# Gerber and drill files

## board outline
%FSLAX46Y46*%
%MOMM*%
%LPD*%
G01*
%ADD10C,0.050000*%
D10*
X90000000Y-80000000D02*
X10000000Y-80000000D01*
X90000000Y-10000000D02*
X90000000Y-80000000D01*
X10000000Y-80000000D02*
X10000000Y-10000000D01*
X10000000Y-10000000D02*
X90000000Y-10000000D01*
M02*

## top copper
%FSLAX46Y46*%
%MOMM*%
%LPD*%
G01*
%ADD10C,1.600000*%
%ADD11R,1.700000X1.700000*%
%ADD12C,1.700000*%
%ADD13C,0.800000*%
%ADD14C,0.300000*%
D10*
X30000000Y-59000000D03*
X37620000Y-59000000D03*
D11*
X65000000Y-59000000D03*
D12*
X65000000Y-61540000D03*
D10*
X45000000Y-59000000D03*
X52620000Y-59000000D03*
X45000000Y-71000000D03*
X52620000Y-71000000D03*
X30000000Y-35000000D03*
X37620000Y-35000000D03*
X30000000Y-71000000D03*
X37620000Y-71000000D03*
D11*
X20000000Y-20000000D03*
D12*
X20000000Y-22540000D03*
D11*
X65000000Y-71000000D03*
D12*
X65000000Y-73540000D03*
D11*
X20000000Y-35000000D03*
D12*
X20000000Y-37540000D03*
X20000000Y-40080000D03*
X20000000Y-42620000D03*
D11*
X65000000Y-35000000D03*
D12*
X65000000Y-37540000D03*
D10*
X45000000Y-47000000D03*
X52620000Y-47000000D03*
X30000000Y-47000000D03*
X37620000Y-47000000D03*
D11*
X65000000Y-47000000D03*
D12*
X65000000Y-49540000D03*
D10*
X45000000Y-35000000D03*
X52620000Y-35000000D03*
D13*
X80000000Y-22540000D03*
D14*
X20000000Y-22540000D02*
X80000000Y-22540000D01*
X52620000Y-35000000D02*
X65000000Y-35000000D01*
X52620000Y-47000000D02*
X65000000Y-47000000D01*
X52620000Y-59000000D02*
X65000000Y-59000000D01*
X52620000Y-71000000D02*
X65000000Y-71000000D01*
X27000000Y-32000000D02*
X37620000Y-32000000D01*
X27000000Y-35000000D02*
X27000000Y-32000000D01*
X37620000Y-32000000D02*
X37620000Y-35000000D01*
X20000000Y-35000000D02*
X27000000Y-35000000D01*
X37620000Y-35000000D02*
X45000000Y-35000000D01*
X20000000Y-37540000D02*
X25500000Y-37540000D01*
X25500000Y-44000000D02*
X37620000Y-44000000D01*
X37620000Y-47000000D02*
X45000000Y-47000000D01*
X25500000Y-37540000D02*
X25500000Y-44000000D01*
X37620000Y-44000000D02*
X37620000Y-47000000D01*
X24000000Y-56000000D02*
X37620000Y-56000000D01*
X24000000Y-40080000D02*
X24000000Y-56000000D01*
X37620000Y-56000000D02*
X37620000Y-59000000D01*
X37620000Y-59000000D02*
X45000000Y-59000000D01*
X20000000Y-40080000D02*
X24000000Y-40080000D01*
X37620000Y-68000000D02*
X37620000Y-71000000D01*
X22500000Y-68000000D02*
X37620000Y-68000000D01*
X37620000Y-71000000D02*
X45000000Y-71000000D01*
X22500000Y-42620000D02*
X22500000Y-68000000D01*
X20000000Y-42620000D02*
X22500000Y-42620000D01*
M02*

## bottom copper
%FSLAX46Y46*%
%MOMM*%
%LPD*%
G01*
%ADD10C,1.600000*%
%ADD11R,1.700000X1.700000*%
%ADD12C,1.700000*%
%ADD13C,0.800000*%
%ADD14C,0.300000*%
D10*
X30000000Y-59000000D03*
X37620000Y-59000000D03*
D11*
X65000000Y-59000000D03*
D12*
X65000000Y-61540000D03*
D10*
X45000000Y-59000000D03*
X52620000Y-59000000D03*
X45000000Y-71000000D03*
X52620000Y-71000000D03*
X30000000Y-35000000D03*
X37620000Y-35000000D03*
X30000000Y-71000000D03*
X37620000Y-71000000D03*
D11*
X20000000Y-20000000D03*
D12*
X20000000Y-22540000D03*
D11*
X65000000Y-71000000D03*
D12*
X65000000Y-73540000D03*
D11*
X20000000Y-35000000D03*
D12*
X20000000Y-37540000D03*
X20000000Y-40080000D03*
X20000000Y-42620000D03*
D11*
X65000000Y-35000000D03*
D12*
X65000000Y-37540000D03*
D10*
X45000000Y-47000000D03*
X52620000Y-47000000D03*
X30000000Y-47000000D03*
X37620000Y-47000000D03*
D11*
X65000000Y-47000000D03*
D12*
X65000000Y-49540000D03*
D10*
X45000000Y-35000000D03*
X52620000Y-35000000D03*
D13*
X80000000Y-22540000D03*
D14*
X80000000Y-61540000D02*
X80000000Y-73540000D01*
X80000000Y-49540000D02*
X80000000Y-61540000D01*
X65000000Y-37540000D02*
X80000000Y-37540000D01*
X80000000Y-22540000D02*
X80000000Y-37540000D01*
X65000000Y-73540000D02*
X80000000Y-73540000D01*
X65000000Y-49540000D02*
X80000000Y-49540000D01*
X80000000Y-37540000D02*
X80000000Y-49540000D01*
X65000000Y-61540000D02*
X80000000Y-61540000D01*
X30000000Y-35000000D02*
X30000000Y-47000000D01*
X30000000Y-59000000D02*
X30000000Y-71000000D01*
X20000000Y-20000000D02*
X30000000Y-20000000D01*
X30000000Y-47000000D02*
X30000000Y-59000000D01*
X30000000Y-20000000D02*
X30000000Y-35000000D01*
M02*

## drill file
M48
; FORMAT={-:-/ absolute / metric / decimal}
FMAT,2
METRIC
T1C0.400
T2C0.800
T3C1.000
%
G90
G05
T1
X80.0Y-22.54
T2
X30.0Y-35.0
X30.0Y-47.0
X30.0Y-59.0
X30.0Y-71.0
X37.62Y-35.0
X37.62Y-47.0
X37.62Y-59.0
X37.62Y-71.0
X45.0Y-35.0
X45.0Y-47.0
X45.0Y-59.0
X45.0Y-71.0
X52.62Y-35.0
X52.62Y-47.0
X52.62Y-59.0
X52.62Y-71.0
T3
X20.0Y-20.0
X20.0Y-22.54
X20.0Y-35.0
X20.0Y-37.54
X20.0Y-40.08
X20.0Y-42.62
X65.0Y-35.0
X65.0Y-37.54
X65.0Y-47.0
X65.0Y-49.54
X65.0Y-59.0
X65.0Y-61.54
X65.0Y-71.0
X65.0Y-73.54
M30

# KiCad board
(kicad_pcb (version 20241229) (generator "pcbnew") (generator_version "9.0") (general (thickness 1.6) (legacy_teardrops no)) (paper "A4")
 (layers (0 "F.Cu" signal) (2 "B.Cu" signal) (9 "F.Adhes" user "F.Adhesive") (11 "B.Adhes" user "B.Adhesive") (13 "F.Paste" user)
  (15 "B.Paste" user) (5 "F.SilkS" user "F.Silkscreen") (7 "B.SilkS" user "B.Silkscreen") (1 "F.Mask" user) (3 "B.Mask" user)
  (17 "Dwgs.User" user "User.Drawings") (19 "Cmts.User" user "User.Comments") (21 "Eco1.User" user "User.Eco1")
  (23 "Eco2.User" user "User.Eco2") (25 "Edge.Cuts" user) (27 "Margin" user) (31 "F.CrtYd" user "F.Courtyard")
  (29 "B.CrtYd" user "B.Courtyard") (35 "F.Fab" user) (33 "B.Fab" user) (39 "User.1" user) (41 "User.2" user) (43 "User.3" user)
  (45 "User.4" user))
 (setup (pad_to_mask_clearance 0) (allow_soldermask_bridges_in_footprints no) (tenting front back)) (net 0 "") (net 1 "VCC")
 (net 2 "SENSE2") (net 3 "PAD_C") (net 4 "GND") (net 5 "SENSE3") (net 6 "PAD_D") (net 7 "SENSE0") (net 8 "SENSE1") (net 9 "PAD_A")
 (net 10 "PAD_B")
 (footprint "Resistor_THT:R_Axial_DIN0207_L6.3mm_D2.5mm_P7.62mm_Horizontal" (layer "F.Cu") (at 30 59)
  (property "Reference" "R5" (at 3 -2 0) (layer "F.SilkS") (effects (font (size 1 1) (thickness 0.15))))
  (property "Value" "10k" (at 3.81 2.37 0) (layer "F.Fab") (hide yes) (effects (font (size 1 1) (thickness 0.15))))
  (pad "1" thru_hole circle (at 0 0) (size 1.6 1.6) (drill 0.8) (layers "*.Cu" "*.Mask") (remove_unused_layers no) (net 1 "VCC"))
  (pad "2" thru_hole circle (at 7.62 0) (size 1.6 1.6) (drill 0.8) (layers "*.Cu" "*.Mask") (remove_unused_layers no) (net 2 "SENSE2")))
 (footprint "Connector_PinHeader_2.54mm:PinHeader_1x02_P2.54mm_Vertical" (layer "F.Cu") (at 65 59)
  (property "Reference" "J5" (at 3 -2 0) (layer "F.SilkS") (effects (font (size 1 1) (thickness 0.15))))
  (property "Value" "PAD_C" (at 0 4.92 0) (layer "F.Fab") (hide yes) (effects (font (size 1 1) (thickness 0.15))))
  (pad "1" thru_hole rect (at 0 0) (size 1.7 1.7) (drill 1) (layers "*.Cu" "*.Mask") (remove_unused_layers no) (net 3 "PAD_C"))
  (pad "2" thru_hole circle (at 0 2.54) (size 1.7 1.7) (drill 1) (layers "*.Cu" "*.Mask") (remove_unused_layers no) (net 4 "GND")))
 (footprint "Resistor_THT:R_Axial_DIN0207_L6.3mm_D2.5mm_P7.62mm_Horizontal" (layer "F.Cu") (at 45 59)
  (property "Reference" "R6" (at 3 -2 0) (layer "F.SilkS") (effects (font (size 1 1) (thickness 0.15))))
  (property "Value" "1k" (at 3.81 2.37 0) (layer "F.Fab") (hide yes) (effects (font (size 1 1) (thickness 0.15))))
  (pad "1" thru_hole circle (at 0 0) (size 1.6 1.6) (drill 0.8) (layers "*.Cu" "*.Mask") (remove_unused_layers no) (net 2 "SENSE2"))
  (pad "2" thru_hole circle (at 7.62 0) (size 1.6 1.6) (drill 0.8) (layers "*.Cu" "*.Mask") (remove_unused_layers no) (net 3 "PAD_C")))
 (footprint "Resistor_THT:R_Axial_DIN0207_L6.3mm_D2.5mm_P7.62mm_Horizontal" (layer "F.Cu") (at 45 71)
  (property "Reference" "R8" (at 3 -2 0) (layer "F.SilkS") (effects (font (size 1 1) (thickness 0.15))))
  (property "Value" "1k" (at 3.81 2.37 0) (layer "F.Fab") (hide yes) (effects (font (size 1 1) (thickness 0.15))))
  (pad "1" thru_hole circle (at 0 0) (size 1.6 1.6) (drill 0.8) (layers "*.Cu" "*.Mask") (remove_unused_layers no) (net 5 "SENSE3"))
  (pad "2" thru_hole circle (at 7.62 0) (size 1.6 1.6) (drill 0.8) (layers "*.Cu" "*.Mask") (remove_unused_layers no) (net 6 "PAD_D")))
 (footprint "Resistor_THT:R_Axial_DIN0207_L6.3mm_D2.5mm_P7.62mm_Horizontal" (layer "F.Cu") (at 30 35)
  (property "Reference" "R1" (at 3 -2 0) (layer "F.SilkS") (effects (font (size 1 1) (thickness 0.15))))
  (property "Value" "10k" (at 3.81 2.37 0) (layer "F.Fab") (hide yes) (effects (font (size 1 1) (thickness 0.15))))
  (pad "1" thru_hole circle (at 0 0) (size 1.6 1.6) (drill 0.8) (layers "*.Cu" "*.Mask") (remove_unused_layers no) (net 1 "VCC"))
  (pad "2" thru_hole circle (at 7.62 0) (size 1.6 1.6) (drill 0.8) (layers "*.Cu" "*.Mask") (remove_unused_layers no) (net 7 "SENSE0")))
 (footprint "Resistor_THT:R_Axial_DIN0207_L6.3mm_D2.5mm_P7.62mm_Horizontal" (layer "F.Cu") (at 30 71)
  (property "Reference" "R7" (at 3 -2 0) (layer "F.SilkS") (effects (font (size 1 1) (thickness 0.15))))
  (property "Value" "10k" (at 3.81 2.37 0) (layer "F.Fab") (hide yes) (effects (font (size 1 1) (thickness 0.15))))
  (pad "1" thru_hole circle (at 0 0) (size 1.6 1.6) (drill 0.8) (layers "*.Cu" "*.Mask") (remove_unused_layers no) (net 1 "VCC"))
  (pad "2" thru_hole circle (at 7.62 0) (size 1.6 1.6) (drill 0.8) (layers "*.Cu" "*.Mask") (remove_unused_layers no) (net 5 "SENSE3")))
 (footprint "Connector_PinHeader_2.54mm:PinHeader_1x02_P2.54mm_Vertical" (layer "F.Cu") (at 20 20)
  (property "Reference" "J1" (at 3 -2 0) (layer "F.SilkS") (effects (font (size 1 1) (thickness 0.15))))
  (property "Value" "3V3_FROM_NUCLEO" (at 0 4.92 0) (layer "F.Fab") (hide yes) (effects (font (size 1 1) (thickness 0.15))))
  (pad "1" thru_hole rect (at 0 0) (size 1.7 1.7) (drill 1) (layers "*.Cu" "*.Mask") (remove_unused_layers no) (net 1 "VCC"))
  (pad "2" thru_hole circle (at 0 2.54) (size 1.7 1.7) (drill 1) (layers "*.Cu" "*.Mask") (remove_unused_layers no) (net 4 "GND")))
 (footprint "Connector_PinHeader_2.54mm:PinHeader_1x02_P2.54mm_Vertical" (layer "F.Cu") (at 65 71)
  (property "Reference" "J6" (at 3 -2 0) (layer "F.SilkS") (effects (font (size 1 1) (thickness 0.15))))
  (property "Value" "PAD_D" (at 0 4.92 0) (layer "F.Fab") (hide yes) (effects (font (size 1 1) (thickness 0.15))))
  (pad "1" thru_hole rect (at 0 0) (size 1.7 1.7) (drill 1) (layers "*.Cu" "*.Mask") (remove_unused_layers no) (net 6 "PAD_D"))
  (pad "2" thru_hole circle (at 0 2.54) (size 1.7 1.7) (drill 1) (layers "*.Cu" "*.Mask") (remove_unused_layers no) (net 4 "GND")))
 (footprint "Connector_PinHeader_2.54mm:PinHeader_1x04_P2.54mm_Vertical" (layer "F.Cu") (at 20 35)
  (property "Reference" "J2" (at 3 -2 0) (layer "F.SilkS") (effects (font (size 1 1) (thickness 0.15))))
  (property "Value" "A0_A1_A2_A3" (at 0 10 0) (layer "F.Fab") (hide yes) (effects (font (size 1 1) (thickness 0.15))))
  (pad "1" thru_hole rect (at 0 0) (size 1.7 1.7) (drill 1) (layers "*.Cu" "*.Mask") (remove_unused_layers no) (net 7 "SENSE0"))
  (pad "2" thru_hole circle (at 0 2.54) (size 1.7 1.7) (drill 1) (layers "*.Cu" "*.Mask") (remove_unused_layers no) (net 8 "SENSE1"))
  (pad "3" thru_hole circle (at 0 5.08) (size 1.7 1.7) (drill 1) (layers "*.Cu" "*.Mask") (remove_unused_layers no) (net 2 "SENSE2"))
  (pad "4" thru_hole circle (at 0 7.62) (size 1.7 1.7) (drill 1) (layers "*.Cu" "*.Mask") (remove_unused_layers no) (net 5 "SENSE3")))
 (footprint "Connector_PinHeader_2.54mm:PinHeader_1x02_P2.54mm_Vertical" (layer "F.Cu") (at 65 35)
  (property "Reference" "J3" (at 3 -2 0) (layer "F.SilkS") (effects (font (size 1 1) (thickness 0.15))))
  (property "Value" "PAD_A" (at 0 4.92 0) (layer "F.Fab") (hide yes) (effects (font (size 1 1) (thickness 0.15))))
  (pad "1" thru_hole rect (at 0 0) (size 1.7 1.7) (drill 1) (layers "*.Cu" "*.Mask") (remove_unused_layers no) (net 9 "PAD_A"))
  (pad "2" thru_hole circle (at 0 2.54) (size 1.7 1.7) (drill 1) (layers "*.Cu" "*.Mask") (remove_unused_layers no) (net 4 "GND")))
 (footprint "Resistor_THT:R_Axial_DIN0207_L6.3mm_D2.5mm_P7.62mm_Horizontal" (layer "F.Cu") (at 45 47)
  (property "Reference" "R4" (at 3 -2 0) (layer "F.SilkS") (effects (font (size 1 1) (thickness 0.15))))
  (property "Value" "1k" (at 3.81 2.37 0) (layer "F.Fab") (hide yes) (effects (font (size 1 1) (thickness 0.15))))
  (pad "1" thru_hole circle (at 0 0) (size 1.6 1.6) (drill 0.8) (layers "*.Cu" "*.Mask") (remove_unused_layers no) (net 8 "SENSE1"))
  (pad "2" thru_hole circle (at 7.62 0) (size 1.6 1.6) (drill 0.8) (layers "*.Cu" "*.Mask") (remove_unused_layers no) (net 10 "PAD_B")))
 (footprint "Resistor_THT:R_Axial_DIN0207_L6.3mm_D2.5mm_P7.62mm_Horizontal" (layer "F.Cu") (at 30 47)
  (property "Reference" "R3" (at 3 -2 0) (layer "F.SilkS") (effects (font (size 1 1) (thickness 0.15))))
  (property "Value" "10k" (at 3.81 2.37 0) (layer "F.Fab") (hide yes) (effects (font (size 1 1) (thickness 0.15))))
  (pad "1" thru_hole circle (at 0 0) (size 1.6 1.6) (drill 0.8) (layers "*.Cu" "*.Mask") (remove_unused_layers no) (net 1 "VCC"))
  (pad "2" thru_hole circle (at 7.62 0) (size 1.6 1.6) (drill 0.8) (layers "*.Cu" "*.Mask") (remove_unused_layers no) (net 8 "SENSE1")))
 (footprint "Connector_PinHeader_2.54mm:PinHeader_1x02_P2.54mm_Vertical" (layer "F.Cu") (at 65 47)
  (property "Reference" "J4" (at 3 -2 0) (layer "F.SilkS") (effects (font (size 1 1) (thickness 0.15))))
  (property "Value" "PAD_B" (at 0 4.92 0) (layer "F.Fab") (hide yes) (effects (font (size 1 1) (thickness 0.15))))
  (pad "1" thru_hole rect (at 0 0) (size 1.7 1.7) (drill 1) (layers "*.Cu" "*.Mask") (remove_unused_layers no) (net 10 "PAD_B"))
  (pad "2" thru_hole circle (at 0 2.54) (size 1.7 1.7) (drill 1) (layers "*.Cu" "*.Mask") (remove_unused_layers no) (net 4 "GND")))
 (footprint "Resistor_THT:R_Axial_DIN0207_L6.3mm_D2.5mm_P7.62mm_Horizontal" (layer "F.Cu") (at 45 35)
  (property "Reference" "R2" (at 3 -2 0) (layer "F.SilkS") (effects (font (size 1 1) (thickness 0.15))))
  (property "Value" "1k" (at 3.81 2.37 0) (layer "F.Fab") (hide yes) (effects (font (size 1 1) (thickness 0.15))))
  (pad "1" thru_hole circle (at 0 0) (size 1.6 1.6) (drill 0.8) (layers "*.Cu" "*.Mask") (remove_unused_layers no) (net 7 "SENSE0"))
  (pad "2" thru_hole circle (at 7.62 0) (size 1.6 1.6) (drill 0.8) (layers "*.Cu" "*.Mask") (remove_unused_layers no) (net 9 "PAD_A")))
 (gr_line (start 90 80) (end 10 80) (stroke (width 0.05) (type default)) (layer "Edge.Cuts"))
 (gr_line (start 90 10) (end 90 80) (stroke (width 0.05) (type default)) (layer "Edge.Cuts"))
 (gr_line (start 10 80) (end 10 10) (stroke (width 0.05) (type default)) (layer "Edge.Cuts"))
 (gr_line (start 10 10) (end 90 10) (stroke (width 0.05) (type default)) (layer "Edge.Cuts"))
 (segment (start 20 22.54) (end 80 22.54) (width 0.3) (layer "F.Cu") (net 4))
 (via (at 80 22.54) (size 0.8) (drill 0.4) (layers "F.Cu" "B.Cu") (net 4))
 (segment (start 80 61.54) (end 80 73.54) (width 0.3) (layer "B.Cu") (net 4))
 (segment (start 80 49.54) (end 80 61.54) (width 0.3) (layer "B.Cu") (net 4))
 (segment (start 65 37.54) (end 80 37.54) (width 0.3) (layer "B.Cu") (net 4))
 (segment (start 80 22.54) (end 80 37.54) (width 0.3) (layer "B.Cu") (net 4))
 (segment (start 65 73.54) (end 80 73.54) (width 0.3) (layer "B.Cu") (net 4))
 (segment (start 65 49.54) (end 80 49.54) (width 0.3) (layer "B.Cu") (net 4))
 (segment (start 80 37.54) (end 80 49.54) (width 0.3) (layer "B.Cu") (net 4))
 (segment (start 65 61.54) (end 80 61.54) (width 0.3) (layer "B.Cu") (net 4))
 (segment (start 52.62 35) (end 65 35) (width 0.3) (layer "F.Cu") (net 9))
 (segment (start 52.62 47) (end 65 47) (width 0.3) (layer "F.Cu") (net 10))
 (segment (start 52.62 59) (end 65 59) (width 0.3) (layer "F.Cu") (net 3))
 (segment (start 52.62 71) (end 65 71) (width 0.3) (layer "F.Cu") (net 6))
 (segment (start 27 32) (end 37.62 32) (width 0.3) (layer "F.Cu") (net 7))
 (segment (start 27 35) (end 27 32) (width 0.3) (layer "F.Cu") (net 7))
 (segment (start 37.62 32) (end 37.62 35) (width 0.3) (layer "F.Cu") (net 7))
 (segment (start 20 35) (end 27 35) (width 0.3) (layer "F.Cu") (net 7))
 (segment (start 37.62 35) (end 45 35) (width 0.3) (layer "F.Cu") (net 7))
 (segment (start 20 37.54) (end 25.5 37.54) (width 0.3) (layer "F.Cu") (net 8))
 (segment (start 25.5 44) (end 37.62 44) (width 0.3) (layer "F.Cu") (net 8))
 (segment (start 37.62 47) (end 45 47) (width 0.3) (layer "F.Cu") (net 8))
 (segment (start 25.5 37.54) (end 25.5 44) (width 0.3) (layer "F.Cu") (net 8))
 (segment (start 37.62 44) (end 37.62 47) (width 0.3) (layer "F.Cu") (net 8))
 (segment (start 24 56) (end 37.62 56) (width 0.3) (layer "F.Cu") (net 2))
 (segment (start 24 40.08) (end 24 56) (width 0.3) (layer "F.Cu") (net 2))
 (segment (start 37.62 56) (end 37.62 59) (width 0.3) (layer "F.Cu") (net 2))
 (segment (start 37.62 59) (end 45 59) (width 0.3) (layer "F.Cu") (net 2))
 (segment (start 20 40.08) (end 24 40.08) (width 0.3) (layer "F.Cu") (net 2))
 (segment (start 37.62 68) (end 37.62 71) (width 0.3) (layer "F.Cu") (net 5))
 (segment (start 22.5 68) (end 37.62 68) (width 0.3) (layer "F.Cu") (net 5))
 (segment (start 37.62 71) (end 45 71) (width 0.3) (layer "F.Cu") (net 5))
 (segment (start 22.5 42.62) (end 22.5 68) (width 0.3) (layer "F.Cu") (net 5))
 (segment (start 20 42.62) (end 22.5 42.62) (width 0.3) (layer "F.Cu") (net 5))
 (segment (start 30 35) (end 30 47) (width 0.3) (layer "B.Cu") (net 1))
 (segment (start 30 59) (end 30 71) (width 0.3) (layer "B.Cu") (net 1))
 (segment (start 20 20) (end 30 20) (width 0.3) (layer "B.Cu") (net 1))
 (segment (start 30 47) (end 30 59) (width 0.3) (layer "B.Cu") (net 1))
 (segment (start 30 20) (end 30 35) (width 0.3) (layer "B.Cu") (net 1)))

